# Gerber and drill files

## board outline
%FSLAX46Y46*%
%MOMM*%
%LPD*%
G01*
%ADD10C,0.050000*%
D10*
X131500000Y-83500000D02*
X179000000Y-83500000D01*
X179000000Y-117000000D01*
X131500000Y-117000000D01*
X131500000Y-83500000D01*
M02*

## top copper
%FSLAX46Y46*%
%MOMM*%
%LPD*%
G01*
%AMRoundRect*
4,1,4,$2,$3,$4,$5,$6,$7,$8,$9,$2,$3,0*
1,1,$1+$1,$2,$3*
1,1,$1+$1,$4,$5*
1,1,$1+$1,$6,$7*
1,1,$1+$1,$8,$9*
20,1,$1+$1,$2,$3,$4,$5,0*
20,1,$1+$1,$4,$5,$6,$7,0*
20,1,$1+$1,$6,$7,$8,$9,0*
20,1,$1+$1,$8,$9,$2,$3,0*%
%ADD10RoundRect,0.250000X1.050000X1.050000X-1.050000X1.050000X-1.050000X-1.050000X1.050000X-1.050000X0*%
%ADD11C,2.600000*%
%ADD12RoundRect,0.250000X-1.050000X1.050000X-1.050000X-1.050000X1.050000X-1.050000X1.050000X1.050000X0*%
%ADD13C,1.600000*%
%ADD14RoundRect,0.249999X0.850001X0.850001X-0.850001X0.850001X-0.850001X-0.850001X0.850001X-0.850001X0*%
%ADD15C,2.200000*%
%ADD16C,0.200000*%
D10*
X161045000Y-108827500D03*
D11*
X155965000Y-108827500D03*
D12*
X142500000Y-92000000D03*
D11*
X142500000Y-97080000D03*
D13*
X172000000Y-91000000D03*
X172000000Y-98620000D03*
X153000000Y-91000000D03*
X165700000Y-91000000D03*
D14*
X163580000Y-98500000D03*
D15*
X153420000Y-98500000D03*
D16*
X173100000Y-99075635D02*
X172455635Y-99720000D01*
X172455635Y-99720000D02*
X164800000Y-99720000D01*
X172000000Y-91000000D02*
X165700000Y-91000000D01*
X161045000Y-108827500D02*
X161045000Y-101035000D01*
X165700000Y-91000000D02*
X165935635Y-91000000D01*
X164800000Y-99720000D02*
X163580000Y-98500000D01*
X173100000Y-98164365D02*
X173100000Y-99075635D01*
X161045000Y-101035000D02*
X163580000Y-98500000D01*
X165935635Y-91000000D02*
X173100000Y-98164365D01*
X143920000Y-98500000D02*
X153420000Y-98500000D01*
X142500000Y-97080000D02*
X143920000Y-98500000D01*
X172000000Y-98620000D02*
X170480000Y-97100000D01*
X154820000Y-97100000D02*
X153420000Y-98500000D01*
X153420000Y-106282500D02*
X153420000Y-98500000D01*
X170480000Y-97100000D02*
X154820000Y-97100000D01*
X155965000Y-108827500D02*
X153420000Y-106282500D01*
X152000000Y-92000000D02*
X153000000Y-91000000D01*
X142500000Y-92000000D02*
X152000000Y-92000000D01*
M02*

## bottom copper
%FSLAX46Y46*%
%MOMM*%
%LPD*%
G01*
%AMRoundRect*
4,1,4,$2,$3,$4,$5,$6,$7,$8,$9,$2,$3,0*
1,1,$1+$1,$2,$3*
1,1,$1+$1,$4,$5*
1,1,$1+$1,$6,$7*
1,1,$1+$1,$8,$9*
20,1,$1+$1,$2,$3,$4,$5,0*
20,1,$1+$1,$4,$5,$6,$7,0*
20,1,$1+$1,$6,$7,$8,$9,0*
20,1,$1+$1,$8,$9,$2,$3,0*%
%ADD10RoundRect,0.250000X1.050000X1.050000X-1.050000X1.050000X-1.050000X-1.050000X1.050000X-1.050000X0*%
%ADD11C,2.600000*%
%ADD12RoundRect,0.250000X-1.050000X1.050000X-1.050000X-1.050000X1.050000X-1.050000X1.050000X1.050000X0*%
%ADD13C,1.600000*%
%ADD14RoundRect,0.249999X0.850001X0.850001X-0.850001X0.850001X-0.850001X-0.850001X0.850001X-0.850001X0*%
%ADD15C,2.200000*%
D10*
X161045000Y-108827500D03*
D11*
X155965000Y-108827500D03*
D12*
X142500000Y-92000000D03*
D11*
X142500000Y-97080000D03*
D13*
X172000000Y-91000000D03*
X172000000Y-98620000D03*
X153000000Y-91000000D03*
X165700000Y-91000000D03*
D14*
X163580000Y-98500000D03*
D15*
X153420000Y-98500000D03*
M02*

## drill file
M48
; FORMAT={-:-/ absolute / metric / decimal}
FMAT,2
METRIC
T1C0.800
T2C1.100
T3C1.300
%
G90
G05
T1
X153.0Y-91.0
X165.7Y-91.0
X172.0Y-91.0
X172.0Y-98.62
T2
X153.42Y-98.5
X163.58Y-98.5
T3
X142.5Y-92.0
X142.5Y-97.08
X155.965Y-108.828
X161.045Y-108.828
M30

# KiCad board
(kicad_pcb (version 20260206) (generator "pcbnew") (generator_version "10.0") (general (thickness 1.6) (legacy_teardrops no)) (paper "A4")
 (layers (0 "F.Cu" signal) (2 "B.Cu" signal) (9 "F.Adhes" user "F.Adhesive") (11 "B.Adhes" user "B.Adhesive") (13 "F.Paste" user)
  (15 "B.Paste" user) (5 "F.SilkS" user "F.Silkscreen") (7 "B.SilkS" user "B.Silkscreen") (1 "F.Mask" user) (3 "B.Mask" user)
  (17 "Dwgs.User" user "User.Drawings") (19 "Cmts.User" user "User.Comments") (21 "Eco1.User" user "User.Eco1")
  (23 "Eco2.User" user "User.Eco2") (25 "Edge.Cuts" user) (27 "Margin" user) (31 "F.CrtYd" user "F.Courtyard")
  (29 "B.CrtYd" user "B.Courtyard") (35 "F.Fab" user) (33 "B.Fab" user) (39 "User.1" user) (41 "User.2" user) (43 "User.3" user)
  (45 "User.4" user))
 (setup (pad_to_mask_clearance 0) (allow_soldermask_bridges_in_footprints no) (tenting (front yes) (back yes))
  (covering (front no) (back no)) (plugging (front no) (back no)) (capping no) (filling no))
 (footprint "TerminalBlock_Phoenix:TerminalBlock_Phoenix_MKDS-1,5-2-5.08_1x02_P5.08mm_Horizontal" (layer "F.Cu") (at 161.045 108.8275 180)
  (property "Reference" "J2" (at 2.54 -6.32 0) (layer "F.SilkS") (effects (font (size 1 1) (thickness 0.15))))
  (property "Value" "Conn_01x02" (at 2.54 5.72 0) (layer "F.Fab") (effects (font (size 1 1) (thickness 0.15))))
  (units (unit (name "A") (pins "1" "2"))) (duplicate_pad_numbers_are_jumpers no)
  (pad "1" thru_hole roundrect (at 0 0 180) (size 2.6 2.6) (drill 1.3) (layers "*.Cu" "*.Mask") (remove_unused_layers no)
   (roundrect_rratio 0.096154) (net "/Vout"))
  (pad "2" thru_hole circle (at 5.08 0 180) (size 2.6 2.6) (drill 1.3) (layers "*.Cu" "*.Mask") (remove_unused_layers no) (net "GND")))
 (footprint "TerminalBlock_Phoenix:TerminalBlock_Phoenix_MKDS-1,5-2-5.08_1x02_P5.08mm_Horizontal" (layer "F.Cu") (at 142.5 92 -90)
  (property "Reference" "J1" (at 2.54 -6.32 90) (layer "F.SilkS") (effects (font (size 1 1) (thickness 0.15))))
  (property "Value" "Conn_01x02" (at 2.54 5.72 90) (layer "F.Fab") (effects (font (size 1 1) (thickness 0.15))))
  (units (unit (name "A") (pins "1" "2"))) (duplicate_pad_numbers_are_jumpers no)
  (pad "1" thru_hole roundrect (at 0 0 270) (size 2.6 2.6) (drill 1.3) (layers "*.Cu" "*.Mask") (remove_unused_layers no)
   (roundrect_rratio 0.096154) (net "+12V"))
  (pad "2" thru_hole circle (at 5.08 0 270) (size 2.6 2.6) (drill 1.3) (layers "*.Cu" "*.Mask") (remove_unused_layers no) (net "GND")))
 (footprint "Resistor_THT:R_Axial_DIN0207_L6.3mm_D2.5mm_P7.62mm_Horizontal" (layer "F.Cu") (at 172 91 -90)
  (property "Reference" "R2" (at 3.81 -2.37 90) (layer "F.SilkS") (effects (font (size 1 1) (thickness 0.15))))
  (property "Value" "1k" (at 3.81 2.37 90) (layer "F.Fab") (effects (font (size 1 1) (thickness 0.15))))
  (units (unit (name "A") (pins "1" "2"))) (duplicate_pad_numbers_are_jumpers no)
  (pad "1" thru_hole circle (at 0 0 270) (size 1.6 1.6) (drill 0.8) (layers "*.Cu" "*.Mask") (remove_unused_layers no) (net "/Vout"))
  (pad "2" thru_hole circle (at 7.62 0 270) (size 1.6 1.6) (drill 0.8) (layers "*.Cu" "*.Mask") (remove_unused_layers no) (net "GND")))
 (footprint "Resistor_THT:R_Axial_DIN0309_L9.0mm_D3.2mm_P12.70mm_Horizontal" (layer "F.Cu") (at 153 91)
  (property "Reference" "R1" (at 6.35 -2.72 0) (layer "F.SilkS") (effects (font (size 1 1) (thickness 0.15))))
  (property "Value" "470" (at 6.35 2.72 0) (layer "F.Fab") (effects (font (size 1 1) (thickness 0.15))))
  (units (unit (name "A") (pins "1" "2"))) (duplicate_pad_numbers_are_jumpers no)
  (pad "1" thru_hole circle (at 0 0) (size 1.6 1.6) (drill 0.8) (layers "*.Cu" "*.Mask") (remove_unused_layers no) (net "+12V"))
  (pad "2" thru_hole circle (at 12.7 0) (size 1.6 1.6) (drill 0.8) (layers "*.Cu" "*.Mask") (remove_unused_layers no) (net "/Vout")))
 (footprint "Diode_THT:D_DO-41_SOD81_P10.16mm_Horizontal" (layer "F.Cu") (at 163.58 98.5 180)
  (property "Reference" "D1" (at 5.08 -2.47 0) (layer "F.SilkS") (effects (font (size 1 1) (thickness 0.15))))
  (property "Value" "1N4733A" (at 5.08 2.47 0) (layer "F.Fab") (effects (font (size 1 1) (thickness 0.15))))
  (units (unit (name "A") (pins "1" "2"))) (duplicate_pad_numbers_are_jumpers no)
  (pad "1" thru_hole roundrect (at 0 0 180) (size 2.2 2.2) (drill 1.1) (layers "*.Cu" "*.Mask") (remove_unused_layers no)
   (roundrect_rratio 0.113636) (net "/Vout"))
  (pad "2" thru_hole circle (at 10.16 0 180) (size 2.2 2.2) (drill 1.1) (layers "*.Cu" "*.Mask") (remove_unused_layers no) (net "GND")))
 (gr_rect (start 131.5 83.5) (end 179 117) (stroke (width 0.05) (type default)) (fill no) (layer "Edge.Cuts"))
 (segment (start 173.1 99.075635) (end 172.455635 99.72) (width 0.2) (layer "F.Cu") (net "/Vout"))
 (segment (start 172.455635 99.72) (end 164.8 99.72) (width 0.2) (layer "F.Cu") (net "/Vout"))
 (segment (start 172 91) (end 165.7 91) (width 0.2) (layer "F.Cu") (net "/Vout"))
 (segment (start 161.045 108.8275) (end 161.045 101.035) (width 0.2) (layer "F.Cu") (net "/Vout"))
 (segment (start 165.7 91) (end 165.935635 91) (width 0.2) (layer "F.Cu") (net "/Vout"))
 (segment (start 164.8 99.72) (end 163.58 98.5) (width 0.2) (layer "F.Cu") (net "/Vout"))
 (segment (start 173.1 98.164365) (end 173.1 99.075635) (width 0.2) (layer "F.Cu") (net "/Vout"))
 (segment (start 161.045 101.035) (end 163.58 98.5) (width 0.2) (layer "F.Cu") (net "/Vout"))
 (segment (start 165.935635 91) (end 173.1 98.164365) (width 0.2) (layer "F.Cu") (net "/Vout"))
 (segment (start 143.92 98.5) (end 153.42 98.5) (width 0.2) (layer "F.Cu") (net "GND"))
 (segment (start 142.5 97.08) (end 143.92 98.5) (width 0.2) (layer "F.Cu") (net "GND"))
 (segment (start 172 98.62) (end 170.48 97.1) (width 0.2) (layer "F.Cu") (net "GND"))
 (segment (start 154.82 97.1) (end 153.42 98.5) (width 0.2) (layer "F.Cu") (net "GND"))
 (segment (start 153.42 106.2825) (end 153.42 98.5) (width 0.2) (layer "F.Cu") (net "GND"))
 (segment (start 170.48 97.1) (end 154.82 97.1) (width 0.2) (layer "F.Cu") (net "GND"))
 (segment (start 155.965 108.8275) (end 153.42 106.2825) (width 0.2) (layer "F.Cu") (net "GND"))
 (segment (start 152 92) (end 153 91) (width 0.2) (layer "F.Cu") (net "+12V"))
 (segment (start 142.5 92) (end 152 92) (width 0.2) (layer "F.Cu") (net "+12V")))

